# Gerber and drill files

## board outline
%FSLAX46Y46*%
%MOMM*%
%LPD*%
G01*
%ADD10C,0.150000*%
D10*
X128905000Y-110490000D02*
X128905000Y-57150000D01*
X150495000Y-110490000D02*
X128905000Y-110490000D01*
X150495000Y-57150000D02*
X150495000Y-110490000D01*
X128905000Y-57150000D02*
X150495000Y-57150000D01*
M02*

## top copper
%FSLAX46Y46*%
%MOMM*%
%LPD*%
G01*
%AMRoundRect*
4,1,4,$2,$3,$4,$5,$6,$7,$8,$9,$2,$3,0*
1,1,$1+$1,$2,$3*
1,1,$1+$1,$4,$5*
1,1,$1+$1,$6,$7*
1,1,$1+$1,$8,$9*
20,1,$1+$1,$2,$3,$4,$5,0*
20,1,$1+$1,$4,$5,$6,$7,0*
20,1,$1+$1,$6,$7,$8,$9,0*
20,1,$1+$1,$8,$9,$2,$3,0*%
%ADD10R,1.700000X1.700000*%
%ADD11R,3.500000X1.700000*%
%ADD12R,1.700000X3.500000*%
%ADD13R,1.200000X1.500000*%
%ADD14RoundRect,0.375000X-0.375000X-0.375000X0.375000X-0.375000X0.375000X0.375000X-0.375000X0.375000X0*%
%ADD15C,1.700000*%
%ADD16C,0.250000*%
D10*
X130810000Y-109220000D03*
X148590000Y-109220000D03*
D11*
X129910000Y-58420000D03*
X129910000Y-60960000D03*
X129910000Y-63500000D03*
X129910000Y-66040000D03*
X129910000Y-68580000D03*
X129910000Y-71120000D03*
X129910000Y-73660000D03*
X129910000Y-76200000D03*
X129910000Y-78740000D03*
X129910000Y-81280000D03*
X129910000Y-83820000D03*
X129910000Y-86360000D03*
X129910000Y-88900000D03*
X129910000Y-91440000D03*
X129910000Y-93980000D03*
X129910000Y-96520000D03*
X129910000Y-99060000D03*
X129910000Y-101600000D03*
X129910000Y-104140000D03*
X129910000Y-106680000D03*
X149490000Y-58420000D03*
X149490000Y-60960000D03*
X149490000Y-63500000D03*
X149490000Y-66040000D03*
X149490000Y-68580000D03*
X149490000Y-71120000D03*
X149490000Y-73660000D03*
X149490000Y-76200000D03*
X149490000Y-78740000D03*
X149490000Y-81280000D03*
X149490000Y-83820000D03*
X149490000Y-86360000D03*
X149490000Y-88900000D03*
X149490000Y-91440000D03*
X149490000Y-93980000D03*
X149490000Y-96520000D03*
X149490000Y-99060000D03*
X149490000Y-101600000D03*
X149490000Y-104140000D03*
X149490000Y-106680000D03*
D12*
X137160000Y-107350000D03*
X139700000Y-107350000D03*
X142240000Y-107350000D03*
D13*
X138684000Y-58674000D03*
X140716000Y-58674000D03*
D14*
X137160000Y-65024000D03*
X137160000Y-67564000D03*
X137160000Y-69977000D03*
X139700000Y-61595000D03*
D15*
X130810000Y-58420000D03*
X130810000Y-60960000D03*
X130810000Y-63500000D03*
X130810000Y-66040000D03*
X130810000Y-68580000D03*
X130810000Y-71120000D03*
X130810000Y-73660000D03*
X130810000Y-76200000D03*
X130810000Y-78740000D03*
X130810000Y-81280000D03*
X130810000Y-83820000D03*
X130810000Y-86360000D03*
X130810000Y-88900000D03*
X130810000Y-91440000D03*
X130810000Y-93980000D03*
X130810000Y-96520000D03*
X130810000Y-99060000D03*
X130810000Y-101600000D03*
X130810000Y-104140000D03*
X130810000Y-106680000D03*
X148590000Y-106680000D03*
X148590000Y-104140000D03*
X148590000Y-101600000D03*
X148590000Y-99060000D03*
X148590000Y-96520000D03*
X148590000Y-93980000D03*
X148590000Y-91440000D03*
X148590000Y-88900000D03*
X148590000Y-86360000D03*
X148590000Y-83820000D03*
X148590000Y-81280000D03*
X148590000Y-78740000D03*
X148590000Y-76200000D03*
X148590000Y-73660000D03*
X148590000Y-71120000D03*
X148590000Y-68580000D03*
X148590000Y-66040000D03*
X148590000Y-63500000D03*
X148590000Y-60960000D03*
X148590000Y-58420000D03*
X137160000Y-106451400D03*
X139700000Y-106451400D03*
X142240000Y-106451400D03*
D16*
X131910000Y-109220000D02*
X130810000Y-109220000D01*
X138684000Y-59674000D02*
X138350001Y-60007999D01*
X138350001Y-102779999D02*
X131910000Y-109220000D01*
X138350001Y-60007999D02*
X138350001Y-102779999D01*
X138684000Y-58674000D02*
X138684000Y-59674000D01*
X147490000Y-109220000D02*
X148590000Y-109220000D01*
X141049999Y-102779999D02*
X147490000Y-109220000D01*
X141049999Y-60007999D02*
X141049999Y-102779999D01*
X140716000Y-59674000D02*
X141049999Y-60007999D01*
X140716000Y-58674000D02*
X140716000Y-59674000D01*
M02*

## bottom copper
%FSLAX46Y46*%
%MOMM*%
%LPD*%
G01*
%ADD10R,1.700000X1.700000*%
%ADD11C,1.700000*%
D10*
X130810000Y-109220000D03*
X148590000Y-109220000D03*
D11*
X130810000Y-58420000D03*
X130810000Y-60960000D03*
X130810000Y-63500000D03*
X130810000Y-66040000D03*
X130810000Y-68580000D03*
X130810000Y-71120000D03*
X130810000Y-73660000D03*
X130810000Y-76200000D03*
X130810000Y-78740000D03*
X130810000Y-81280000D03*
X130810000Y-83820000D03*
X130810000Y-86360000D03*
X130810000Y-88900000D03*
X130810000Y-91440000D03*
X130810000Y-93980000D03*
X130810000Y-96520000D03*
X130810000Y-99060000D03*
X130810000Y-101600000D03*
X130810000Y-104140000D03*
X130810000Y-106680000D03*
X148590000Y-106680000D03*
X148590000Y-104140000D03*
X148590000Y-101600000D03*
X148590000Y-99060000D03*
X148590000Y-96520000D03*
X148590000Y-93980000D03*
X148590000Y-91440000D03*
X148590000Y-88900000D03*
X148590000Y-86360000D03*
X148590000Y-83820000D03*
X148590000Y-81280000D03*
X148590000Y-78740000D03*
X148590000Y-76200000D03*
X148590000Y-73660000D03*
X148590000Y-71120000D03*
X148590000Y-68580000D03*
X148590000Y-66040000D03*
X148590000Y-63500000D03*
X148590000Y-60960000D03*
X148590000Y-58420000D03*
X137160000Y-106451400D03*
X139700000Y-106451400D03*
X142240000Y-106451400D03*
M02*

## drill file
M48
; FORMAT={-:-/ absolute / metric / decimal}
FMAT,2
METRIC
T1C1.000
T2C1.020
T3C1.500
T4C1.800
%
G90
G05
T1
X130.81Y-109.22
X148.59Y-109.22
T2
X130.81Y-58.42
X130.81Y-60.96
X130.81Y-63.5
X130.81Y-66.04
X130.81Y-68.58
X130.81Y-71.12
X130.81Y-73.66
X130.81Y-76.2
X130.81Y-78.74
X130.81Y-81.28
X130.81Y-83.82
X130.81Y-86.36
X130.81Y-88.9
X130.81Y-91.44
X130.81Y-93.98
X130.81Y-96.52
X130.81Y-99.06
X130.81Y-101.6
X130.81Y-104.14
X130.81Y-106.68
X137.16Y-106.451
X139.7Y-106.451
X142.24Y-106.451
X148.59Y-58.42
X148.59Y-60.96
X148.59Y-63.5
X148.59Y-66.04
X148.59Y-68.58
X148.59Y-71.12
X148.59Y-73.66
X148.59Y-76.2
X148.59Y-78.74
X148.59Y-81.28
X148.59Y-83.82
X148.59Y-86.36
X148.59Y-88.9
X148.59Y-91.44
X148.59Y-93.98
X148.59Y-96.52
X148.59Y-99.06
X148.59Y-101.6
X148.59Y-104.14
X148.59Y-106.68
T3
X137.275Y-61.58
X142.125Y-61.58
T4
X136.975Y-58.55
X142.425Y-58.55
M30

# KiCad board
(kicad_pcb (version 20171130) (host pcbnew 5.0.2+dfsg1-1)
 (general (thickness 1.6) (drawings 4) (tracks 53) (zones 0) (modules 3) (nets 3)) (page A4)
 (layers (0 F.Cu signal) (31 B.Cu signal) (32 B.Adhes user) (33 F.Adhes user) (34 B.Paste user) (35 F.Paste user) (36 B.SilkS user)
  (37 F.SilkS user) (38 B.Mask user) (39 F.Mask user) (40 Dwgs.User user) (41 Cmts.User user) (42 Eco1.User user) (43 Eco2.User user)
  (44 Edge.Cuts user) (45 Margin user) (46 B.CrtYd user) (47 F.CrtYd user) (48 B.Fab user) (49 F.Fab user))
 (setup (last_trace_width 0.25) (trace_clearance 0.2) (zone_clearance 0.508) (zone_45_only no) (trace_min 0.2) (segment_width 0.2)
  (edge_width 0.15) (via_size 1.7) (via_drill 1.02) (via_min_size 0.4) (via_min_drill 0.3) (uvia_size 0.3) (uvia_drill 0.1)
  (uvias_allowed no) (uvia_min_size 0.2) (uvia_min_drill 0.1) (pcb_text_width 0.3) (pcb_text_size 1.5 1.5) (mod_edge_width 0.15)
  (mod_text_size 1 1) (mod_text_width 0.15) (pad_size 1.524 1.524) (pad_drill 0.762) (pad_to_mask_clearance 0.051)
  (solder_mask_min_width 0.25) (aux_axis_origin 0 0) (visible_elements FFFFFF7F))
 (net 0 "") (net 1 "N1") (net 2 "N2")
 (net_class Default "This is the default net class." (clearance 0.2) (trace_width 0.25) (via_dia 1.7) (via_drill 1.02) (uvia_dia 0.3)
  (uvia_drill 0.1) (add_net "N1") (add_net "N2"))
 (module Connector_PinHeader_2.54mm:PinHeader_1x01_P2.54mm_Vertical (layer F.Cu) (at 130.81 109.22)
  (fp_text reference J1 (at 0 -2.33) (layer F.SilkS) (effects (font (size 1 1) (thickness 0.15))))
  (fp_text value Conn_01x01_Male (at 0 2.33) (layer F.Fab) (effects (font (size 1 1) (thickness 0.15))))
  (pad 1 thru_hole rect (at 0 0) (size 1.7 1.7) (drill 1) (layers *.Cu *.Mask) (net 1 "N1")))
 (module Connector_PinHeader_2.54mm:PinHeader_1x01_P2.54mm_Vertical (layer F.Cu) (at 148.59 109.22)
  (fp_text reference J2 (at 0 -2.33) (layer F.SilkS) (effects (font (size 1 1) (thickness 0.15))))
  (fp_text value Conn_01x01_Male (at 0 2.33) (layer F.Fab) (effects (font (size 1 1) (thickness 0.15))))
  (pad 1 thru_hole rect (at 0 0) (size 1.7 1.7) (drill 1) (layers *.Cu *.Mask) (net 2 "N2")))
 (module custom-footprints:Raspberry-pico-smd (layer F.Cu) (at 139.7 82.55)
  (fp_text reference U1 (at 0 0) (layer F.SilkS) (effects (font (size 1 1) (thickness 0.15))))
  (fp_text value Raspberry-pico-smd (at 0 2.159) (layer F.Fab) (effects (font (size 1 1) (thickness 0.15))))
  (pad 1 smd rect (at -8.89 -24.13) (size 3.5 1.7) (drill (offset -0.9 0)) (layers F.Cu F.Mask))
  (pad 2 smd rect (at -8.89 -21.59) (size 3.5 1.7) (drill (offset -0.9 0)) (layers F.Cu F.Mask))
  (pad 3 smd rect (at -8.89 -19.05) (size 3.5 1.7) (drill (offset -0.9 0)) (layers F.Cu F.Mask))
  (pad 4 smd rect (at -8.89 -16.51) (size 3.5 1.7) (drill (offset -0.9 0)) (layers F.Cu F.Mask))
  (pad 5 smd rect (at -8.89 -13.97) (size 3.5 1.7) (drill (offset -0.9 0)) (layers F.Cu F.Mask))
  (pad 6 smd rect (at -8.89 -11.43) (size 3.5 1.7) (drill (offset -0.9 0)) (layers F.Cu F.Mask))
  (pad 7 smd rect (at -8.89 -8.89) (size 3.5 1.7) (drill (offset -0.9 0)) (layers F.Cu F.Mask))
  (pad 8 smd rect (at -8.89 -6.35) (size 3.5 1.7) (drill (offset -0.9 0)) (layers F.Cu F.Mask))
  (pad 9 smd rect (at -8.89 -3.81) (size 3.5 1.7) (drill (offset -0.9 0)) (layers F.Cu F.Mask))
  (pad 10 smd rect (at -8.89 -1.27) (size 3.5 1.7) (drill (offset -0.9 0)) (layers F.Cu F.Mask))
  (pad 11 smd rect (at -8.89 1.27) (size 3.5 1.7) (drill (offset -0.9 0)) (layers F.Cu F.Mask))
  (pad 12 smd rect (at -8.89 3.81) (size 3.5 1.7) (drill (offset -0.9 0)) (layers F.Cu F.Mask))
  (pad 13 smd rect (at -8.89 6.35) (size 3.5 1.7) (drill (offset -0.9 0)) (layers F.Cu F.Mask))
  (pad 14 smd rect (at -8.89 8.89) (size 3.5 1.7) (drill (offset -0.9 0)) (layers F.Cu F.Mask))
  (pad 15 smd rect (at -8.89 11.43) (size 3.5 1.7) (drill (offset -0.9 0)) (layers F.Cu F.Mask))
  (pad 16 smd rect (at -8.89 13.97) (size 3.5 1.7) (drill (offset -0.9 0)) (layers F.Cu F.Mask))
  (pad 17 smd rect (at -8.89 16.51) (size 3.5 1.7) (drill (offset -0.9 0)) (layers F.Cu F.Mask))
  (pad 18 smd rect (at -8.89 19.05) (size 3.5 1.7) (drill (offset -0.9 0)) (layers F.Cu F.Mask))
  (pad 19 smd rect (at -8.89 21.59) (size 3.5 1.7) (drill (offset -0.9 0)) (layers F.Cu F.Mask))
  (pad 20 smd rect (at -8.89 24.13) (size 3.5 1.7) (drill (offset -0.9 0)) (layers F.Cu F.Mask))
  (pad 40 smd rect (at 8.89 -24.13) (size 3.5 1.7) (drill (offset 0.9 0)) (layers F.Cu F.Mask))
  (pad 39 smd rect (at 8.89 -21.59) (size 3.5 1.7) (drill (offset 0.9 0)) (layers F.Cu F.Mask))
  (pad 38 smd rect (at 8.89 -19.05) (size 3.5 1.7) (drill (offset 0.9 0)) (layers F.Cu F.Mask))
  (pad 37 smd rect (at 8.89 -16.51) (size 3.5 1.7) (drill (offset 0.9 0)) (layers F.Cu F.Mask))
  (pad 36 smd rect (at 8.89 -13.97) (size 3.5 1.7) (drill (offset 0.9 0)) (layers F.Cu F.Mask))
  (pad 35 smd rect (at 8.89 -11.43) (size 3.5 1.7) (drill (offset 0.9 0)) (layers F.Cu F.Mask))
  (pad 34 smd rect (at 8.89 -8.89) (size 3.5 1.7) (drill (offset 0.9 0)) (layers F.Cu F.Mask))
  (pad 33 smd rect (at 8.89 -6.35) (size 3.5 1.7) (drill (offset 0.9 0)) (layers F.Cu F.Mask))
  (pad 32 smd rect (at 8.89 -3.81) (size 3.5 1.7) (drill (offset 0.9 0)) (layers F.Cu F.Mask))
  (pad 31 smd rect (at 8.89 -1.27) (size 3.5 1.7) (drill (offset 0.9 0)) (layers F.Cu F.Mask))
  (pad 30 smd rect (at 8.89 1.27) (size 3.5 1.7) (drill (offset 0.9 0)) (layers F.Cu F.Mask))
  (pad 29 smd rect (at 8.89 3.81) (size 3.5 1.7) (drill (offset 0.9 0)) (layers F.Cu F.Mask))
  (pad 28 smd rect (at 8.89 6.35) (size 3.5 1.7) (drill (offset 0.9 0)) (layers F.Cu F.Mask))
  (pad 27 smd rect (at 8.89 8.89) (size 3.5 1.7) (drill (offset 0.9 0)) (layers F.Cu F.Mask))
  (pad 26 smd rect (at 8.89 11.43) (size 3.5 1.7) (drill (offset 0.9 0)) (layers F.Cu F.Mask))
  (pad 25 smd rect (at 8.89 13.97) (size 3.5 1.7) (drill (offset 0.9 0)) (layers F.Cu F.Mask))
  (pad 24 smd rect (at 8.89 16.51) (size 3.5 1.7) (drill (offset 0.9 0)) (layers F.Cu F.Mask))
  (pad 23 smd rect (at 8.89 19.05) (size 3.5 1.7) (drill (offset 0.9 0)) (layers F.Cu F.Mask))
  (pad 22 smd rect (at 8.89 21.59) (size 3.5 1.7) (drill (offset 0.9 0)) (layers F.Cu F.Mask))
  (pad 21 smd rect (at 8.89 24.13) (size 3.5 1.7) (drill (offset 0.9 0)) (layers F.Cu F.Mask))
  (pad "" np_thru_hole oval (at -2.725 -24) (size 1.8 1.8) (drill 1.8) (layers *.Cu *.Mask))
  (pad "" np_thru_hole oval (at 2.725 -24) (size 1.8 1.8) (drill 1.8) (layers *.Cu *.Mask))
  (pad "" np_thru_hole oval (at -2.425 -20.97) (size 1.5 1.5) (drill 1.5) (layers *.Cu *.Mask))
  (pad "" np_thru_hole oval (at 2.425 -20.97) (size 1.5 1.5) (drill 1.5) (layers *.Cu *.Mask))
  (pad 47 smd rect (at -2.54 23.9 90) (size 3.5 1.7) (drill (offset -0.9 0)) (layers F.Cu F.Mask))
  (pad 48 smd rect (at 0 23.9 90) (size 3.5 1.7) (drill (offset -0.9 0)) (layers F.Cu F.Mask))
  (pad 49 smd rect (at 2.54 23.9 90) (size 3.5 1.7) (drill (offset -0.9 0)) (layers F.Cu F.Mask))
  (pad 43 smd rect (at -1.016 -23.876) (size 1.2 1.5) (layers F.Cu F.Mask) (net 1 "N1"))
  (pad 42 smd rect (at 1.016 -23.876) (size 1.2 1.5) (layers F.Cu F.Mask) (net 2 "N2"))
  (pad 44 smd roundrect (at -2.54 -17.526) (size 1.5 1.5) (layers F.Cu F.Mask) (roundrect_rratio 0.25))
  (pad 45 smd roundrect (at -2.54 -14.986) (size 1.5 1.5) (layers F.Cu F.Mask) (roundrect_rratio 0.25))
  (pad 46 smd roundrect (at -2.54 -12.573) (size 1.5 1.5) (layers F.Cu F.Mask) (roundrect_rratio 0.25))
  (pad 41 smd roundrect (at 0 -20.955) (size 1.5 1.5) (layers F.Cu F.Mask) (roundrect_rratio 0.25)))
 (gr_line (start 128.905 110.49) (end 128.905 57.15) (layer Edge.Cuts) (width 0.15))
 (gr_line (start 150.495 110.49) (end 128.905 110.49) (layer Edge.Cuts) (width 0.15))
 (gr_line (start 150.495 57.15) (end 150.495 110.49) (layer Edge.Cuts) (width 0.15))
 (gr_line (start 128.905 57.15) (end 150.495 57.15) (layer Edge.Cuts) (width 0.15))
 (via (at 130.81 58.42) (size 1.7) (drill 1.02) (layers F.Cu B.Cu) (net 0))
 (via (at 130.81 60.96) (size 1.7) (drill 1.02) (layers F.Cu B.Cu) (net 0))
 (via (at 130.81 63.5) (size 1.7) (drill 1.02) (layers F.Cu B.Cu) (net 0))
 (via (at 130.81 66.04) (size 1.7) (drill 1.02) (layers F.Cu B.Cu) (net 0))
 (via (at 130.81 68.58) (size 1.7) (drill 1.02) (layers F.Cu B.Cu) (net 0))
 (via (at 130.81 71.12) (size 1.7) (drill 1.02) (layers F.Cu B.Cu) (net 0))
 (via (at 130.81 73.66) (size 1.7) (drill 1.02) (layers F.Cu B.Cu) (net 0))
 (via (at 130.81 76.2) (size 1.7) (drill 1.02) (layers F.Cu B.Cu) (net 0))
 (via (at 130.81 78.74) (size 1.7) (drill 1.02) (layers F.Cu B.Cu) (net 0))
 (via (at 130.81 81.28) (size 1.7) (drill 1.02) (layers F.Cu B.Cu) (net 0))
 (via (at 130.81 83.82) (size 1.7) (drill 1.02) (layers F.Cu B.Cu) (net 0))
 (via (at 130.81 86.36) (size 1.7) (drill 1.02) (layers F.Cu B.Cu) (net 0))
 (via (at 130.81 88.9) (size 1.7) (drill 1.02) (layers F.Cu B.Cu) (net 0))
 (via (at 130.81 91.44) (size 1.7) (drill 1.02) (layers F.Cu B.Cu) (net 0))
 (via (at 130.81 93.98) (size 1.7) (drill 1.02) (layers F.Cu B.Cu) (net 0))
 (via (at 130.81 96.52) (size 1.7) (drill 1.02) (layers F.Cu B.Cu) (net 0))
 (via (at 130.81 99.06) (size 1.7) (drill 1.02) (layers F.Cu B.Cu) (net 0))
 (via (at 130.81 101.6) (size 1.7) (drill 1.02) (layers F.Cu B.Cu) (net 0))
 (via (at 130.81 104.14) (size 1.7) (drill 1.02) (layers F.Cu B.Cu) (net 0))
 (via (at 130.81 106.68) (size 1.7) (drill 1.02) (layers F.Cu B.Cu) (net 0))
 (via (at 148.59 106.68) (size 1.7) (drill 1.02) (layers F.Cu B.Cu) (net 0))
 (via (at 148.59 104.14) (size 1.7) (drill 1.02) (layers F.Cu B.Cu) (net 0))
 (via (at 148.59 101.6) (size 1.7) (drill 1.02) (layers F.Cu B.Cu) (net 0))
 (via (at 148.59 99.06) (size 1.7) (drill 1.02) (layers F.Cu B.Cu) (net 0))
 (via (at 148.59 96.52) (size 1.7) (drill 1.02) (layers F.Cu B.Cu) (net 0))
 (via (at 148.59 93.98) (size 1.7) (drill 1.02) (layers F.Cu B.Cu) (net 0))
 (via (at 148.59 91.44) (size 1.7) (drill 1.02) (layers F.Cu B.Cu) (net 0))
 (via (at 148.59 88.9) (size 1.7) (drill 1.02) (layers F.Cu B.Cu) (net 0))
 (via (at 148.59 86.36) (size 1.7) (drill 1.02) (layers F.Cu B.Cu) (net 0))
 (via (at 148.59 83.82) (size 1.7) (drill 1.02) (layers F.Cu B.Cu) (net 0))
 (via (at 148.59 81.28) (size 1.7) (drill 1.02) (layers F.Cu B.Cu) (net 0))
 (via (at 148.59 78.74) (size 1.7) (drill 1.02) (layers F.Cu B.Cu) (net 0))
 (via (at 148.59 76.2) (size 1.7) (drill 1.02) (layers F.Cu B.Cu) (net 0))
 (via (at 148.59 73.66) (size 1.7) (drill 1.02) (layers F.Cu B.Cu) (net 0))
 (via (at 148.59 71.12) (size 1.7) (drill 1.02) (layers F.Cu B.Cu) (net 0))
 (via (at 148.59 68.58) (size 1.7) (drill 1.02) (layers F.Cu B.Cu) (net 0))
 (via (at 148.59 66.04) (size 1.7) (drill 1.02) (layers F.Cu B.Cu) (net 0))
 (via (at 148.59 63.5) (size 1.7) (drill 1.02) (layers F.Cu B.Cu) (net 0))
 (via (at 148.59 60.96) (size 1.7) (drill 1.02) (layers F.Cu B.Cu) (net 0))
 (via (at 148.59 58.42) (size 1.7) (drill 1.02) (layers F.Cu B.Cu) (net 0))
 (via (at 137.16 106.4514) (size 1.7) (drill 1.02) (layers F.Cu B.Cu) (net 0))
 (via (at 139.7 106.4514) (size 1.7) (drill 1.02) (layers F.Cu B.Cu) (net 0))
 (via (at 142.24 106.4514) (size 1.7) (drill 1.02) (layers F.Cu B.Cu) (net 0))
 (segment (start 131.91 109.22) (end 130.81 109.22) (width 0.25) (layer F.Cu) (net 1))
 (segment (start 138.684 59.674) (end 138.350001 60.007999) (width 0.25) (layer F.Cu) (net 1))
 (segment (start 138.350001 102.779999) (end 131.91 109.22) (width 0.25) (layer F.Cu) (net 1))
 (segment (start 138.350001 60.007999) (end 138.350001 102.779999) (width 0.25) (layer F.Cu) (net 1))
 (segment (start 138.684 58.674) (end 138.684 59.674) (width 0.25) (layer F.Cu) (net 1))
 (segment (start 147.49 109.22) (end 148.59 109.22) (width 0.25) (layer F.Cu) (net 2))
 (segment (start 141.049999 102.779999) (end 147.49 109.22) (width 0.25) (layer F.Cu) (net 2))
 (segment (start 141.049999 60.007999) (end 141.049999 102.779999) (width 0.25) (layer F.Cu) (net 2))
 (segment (start 140.716 59.674) (end 141.049999 60.007999) (width 0.25) (layer F.Cu) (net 2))
 (segment (start 140.716 58.674) (end 140.716 59.674) (width 0.25) (layer F.Cu) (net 2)))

